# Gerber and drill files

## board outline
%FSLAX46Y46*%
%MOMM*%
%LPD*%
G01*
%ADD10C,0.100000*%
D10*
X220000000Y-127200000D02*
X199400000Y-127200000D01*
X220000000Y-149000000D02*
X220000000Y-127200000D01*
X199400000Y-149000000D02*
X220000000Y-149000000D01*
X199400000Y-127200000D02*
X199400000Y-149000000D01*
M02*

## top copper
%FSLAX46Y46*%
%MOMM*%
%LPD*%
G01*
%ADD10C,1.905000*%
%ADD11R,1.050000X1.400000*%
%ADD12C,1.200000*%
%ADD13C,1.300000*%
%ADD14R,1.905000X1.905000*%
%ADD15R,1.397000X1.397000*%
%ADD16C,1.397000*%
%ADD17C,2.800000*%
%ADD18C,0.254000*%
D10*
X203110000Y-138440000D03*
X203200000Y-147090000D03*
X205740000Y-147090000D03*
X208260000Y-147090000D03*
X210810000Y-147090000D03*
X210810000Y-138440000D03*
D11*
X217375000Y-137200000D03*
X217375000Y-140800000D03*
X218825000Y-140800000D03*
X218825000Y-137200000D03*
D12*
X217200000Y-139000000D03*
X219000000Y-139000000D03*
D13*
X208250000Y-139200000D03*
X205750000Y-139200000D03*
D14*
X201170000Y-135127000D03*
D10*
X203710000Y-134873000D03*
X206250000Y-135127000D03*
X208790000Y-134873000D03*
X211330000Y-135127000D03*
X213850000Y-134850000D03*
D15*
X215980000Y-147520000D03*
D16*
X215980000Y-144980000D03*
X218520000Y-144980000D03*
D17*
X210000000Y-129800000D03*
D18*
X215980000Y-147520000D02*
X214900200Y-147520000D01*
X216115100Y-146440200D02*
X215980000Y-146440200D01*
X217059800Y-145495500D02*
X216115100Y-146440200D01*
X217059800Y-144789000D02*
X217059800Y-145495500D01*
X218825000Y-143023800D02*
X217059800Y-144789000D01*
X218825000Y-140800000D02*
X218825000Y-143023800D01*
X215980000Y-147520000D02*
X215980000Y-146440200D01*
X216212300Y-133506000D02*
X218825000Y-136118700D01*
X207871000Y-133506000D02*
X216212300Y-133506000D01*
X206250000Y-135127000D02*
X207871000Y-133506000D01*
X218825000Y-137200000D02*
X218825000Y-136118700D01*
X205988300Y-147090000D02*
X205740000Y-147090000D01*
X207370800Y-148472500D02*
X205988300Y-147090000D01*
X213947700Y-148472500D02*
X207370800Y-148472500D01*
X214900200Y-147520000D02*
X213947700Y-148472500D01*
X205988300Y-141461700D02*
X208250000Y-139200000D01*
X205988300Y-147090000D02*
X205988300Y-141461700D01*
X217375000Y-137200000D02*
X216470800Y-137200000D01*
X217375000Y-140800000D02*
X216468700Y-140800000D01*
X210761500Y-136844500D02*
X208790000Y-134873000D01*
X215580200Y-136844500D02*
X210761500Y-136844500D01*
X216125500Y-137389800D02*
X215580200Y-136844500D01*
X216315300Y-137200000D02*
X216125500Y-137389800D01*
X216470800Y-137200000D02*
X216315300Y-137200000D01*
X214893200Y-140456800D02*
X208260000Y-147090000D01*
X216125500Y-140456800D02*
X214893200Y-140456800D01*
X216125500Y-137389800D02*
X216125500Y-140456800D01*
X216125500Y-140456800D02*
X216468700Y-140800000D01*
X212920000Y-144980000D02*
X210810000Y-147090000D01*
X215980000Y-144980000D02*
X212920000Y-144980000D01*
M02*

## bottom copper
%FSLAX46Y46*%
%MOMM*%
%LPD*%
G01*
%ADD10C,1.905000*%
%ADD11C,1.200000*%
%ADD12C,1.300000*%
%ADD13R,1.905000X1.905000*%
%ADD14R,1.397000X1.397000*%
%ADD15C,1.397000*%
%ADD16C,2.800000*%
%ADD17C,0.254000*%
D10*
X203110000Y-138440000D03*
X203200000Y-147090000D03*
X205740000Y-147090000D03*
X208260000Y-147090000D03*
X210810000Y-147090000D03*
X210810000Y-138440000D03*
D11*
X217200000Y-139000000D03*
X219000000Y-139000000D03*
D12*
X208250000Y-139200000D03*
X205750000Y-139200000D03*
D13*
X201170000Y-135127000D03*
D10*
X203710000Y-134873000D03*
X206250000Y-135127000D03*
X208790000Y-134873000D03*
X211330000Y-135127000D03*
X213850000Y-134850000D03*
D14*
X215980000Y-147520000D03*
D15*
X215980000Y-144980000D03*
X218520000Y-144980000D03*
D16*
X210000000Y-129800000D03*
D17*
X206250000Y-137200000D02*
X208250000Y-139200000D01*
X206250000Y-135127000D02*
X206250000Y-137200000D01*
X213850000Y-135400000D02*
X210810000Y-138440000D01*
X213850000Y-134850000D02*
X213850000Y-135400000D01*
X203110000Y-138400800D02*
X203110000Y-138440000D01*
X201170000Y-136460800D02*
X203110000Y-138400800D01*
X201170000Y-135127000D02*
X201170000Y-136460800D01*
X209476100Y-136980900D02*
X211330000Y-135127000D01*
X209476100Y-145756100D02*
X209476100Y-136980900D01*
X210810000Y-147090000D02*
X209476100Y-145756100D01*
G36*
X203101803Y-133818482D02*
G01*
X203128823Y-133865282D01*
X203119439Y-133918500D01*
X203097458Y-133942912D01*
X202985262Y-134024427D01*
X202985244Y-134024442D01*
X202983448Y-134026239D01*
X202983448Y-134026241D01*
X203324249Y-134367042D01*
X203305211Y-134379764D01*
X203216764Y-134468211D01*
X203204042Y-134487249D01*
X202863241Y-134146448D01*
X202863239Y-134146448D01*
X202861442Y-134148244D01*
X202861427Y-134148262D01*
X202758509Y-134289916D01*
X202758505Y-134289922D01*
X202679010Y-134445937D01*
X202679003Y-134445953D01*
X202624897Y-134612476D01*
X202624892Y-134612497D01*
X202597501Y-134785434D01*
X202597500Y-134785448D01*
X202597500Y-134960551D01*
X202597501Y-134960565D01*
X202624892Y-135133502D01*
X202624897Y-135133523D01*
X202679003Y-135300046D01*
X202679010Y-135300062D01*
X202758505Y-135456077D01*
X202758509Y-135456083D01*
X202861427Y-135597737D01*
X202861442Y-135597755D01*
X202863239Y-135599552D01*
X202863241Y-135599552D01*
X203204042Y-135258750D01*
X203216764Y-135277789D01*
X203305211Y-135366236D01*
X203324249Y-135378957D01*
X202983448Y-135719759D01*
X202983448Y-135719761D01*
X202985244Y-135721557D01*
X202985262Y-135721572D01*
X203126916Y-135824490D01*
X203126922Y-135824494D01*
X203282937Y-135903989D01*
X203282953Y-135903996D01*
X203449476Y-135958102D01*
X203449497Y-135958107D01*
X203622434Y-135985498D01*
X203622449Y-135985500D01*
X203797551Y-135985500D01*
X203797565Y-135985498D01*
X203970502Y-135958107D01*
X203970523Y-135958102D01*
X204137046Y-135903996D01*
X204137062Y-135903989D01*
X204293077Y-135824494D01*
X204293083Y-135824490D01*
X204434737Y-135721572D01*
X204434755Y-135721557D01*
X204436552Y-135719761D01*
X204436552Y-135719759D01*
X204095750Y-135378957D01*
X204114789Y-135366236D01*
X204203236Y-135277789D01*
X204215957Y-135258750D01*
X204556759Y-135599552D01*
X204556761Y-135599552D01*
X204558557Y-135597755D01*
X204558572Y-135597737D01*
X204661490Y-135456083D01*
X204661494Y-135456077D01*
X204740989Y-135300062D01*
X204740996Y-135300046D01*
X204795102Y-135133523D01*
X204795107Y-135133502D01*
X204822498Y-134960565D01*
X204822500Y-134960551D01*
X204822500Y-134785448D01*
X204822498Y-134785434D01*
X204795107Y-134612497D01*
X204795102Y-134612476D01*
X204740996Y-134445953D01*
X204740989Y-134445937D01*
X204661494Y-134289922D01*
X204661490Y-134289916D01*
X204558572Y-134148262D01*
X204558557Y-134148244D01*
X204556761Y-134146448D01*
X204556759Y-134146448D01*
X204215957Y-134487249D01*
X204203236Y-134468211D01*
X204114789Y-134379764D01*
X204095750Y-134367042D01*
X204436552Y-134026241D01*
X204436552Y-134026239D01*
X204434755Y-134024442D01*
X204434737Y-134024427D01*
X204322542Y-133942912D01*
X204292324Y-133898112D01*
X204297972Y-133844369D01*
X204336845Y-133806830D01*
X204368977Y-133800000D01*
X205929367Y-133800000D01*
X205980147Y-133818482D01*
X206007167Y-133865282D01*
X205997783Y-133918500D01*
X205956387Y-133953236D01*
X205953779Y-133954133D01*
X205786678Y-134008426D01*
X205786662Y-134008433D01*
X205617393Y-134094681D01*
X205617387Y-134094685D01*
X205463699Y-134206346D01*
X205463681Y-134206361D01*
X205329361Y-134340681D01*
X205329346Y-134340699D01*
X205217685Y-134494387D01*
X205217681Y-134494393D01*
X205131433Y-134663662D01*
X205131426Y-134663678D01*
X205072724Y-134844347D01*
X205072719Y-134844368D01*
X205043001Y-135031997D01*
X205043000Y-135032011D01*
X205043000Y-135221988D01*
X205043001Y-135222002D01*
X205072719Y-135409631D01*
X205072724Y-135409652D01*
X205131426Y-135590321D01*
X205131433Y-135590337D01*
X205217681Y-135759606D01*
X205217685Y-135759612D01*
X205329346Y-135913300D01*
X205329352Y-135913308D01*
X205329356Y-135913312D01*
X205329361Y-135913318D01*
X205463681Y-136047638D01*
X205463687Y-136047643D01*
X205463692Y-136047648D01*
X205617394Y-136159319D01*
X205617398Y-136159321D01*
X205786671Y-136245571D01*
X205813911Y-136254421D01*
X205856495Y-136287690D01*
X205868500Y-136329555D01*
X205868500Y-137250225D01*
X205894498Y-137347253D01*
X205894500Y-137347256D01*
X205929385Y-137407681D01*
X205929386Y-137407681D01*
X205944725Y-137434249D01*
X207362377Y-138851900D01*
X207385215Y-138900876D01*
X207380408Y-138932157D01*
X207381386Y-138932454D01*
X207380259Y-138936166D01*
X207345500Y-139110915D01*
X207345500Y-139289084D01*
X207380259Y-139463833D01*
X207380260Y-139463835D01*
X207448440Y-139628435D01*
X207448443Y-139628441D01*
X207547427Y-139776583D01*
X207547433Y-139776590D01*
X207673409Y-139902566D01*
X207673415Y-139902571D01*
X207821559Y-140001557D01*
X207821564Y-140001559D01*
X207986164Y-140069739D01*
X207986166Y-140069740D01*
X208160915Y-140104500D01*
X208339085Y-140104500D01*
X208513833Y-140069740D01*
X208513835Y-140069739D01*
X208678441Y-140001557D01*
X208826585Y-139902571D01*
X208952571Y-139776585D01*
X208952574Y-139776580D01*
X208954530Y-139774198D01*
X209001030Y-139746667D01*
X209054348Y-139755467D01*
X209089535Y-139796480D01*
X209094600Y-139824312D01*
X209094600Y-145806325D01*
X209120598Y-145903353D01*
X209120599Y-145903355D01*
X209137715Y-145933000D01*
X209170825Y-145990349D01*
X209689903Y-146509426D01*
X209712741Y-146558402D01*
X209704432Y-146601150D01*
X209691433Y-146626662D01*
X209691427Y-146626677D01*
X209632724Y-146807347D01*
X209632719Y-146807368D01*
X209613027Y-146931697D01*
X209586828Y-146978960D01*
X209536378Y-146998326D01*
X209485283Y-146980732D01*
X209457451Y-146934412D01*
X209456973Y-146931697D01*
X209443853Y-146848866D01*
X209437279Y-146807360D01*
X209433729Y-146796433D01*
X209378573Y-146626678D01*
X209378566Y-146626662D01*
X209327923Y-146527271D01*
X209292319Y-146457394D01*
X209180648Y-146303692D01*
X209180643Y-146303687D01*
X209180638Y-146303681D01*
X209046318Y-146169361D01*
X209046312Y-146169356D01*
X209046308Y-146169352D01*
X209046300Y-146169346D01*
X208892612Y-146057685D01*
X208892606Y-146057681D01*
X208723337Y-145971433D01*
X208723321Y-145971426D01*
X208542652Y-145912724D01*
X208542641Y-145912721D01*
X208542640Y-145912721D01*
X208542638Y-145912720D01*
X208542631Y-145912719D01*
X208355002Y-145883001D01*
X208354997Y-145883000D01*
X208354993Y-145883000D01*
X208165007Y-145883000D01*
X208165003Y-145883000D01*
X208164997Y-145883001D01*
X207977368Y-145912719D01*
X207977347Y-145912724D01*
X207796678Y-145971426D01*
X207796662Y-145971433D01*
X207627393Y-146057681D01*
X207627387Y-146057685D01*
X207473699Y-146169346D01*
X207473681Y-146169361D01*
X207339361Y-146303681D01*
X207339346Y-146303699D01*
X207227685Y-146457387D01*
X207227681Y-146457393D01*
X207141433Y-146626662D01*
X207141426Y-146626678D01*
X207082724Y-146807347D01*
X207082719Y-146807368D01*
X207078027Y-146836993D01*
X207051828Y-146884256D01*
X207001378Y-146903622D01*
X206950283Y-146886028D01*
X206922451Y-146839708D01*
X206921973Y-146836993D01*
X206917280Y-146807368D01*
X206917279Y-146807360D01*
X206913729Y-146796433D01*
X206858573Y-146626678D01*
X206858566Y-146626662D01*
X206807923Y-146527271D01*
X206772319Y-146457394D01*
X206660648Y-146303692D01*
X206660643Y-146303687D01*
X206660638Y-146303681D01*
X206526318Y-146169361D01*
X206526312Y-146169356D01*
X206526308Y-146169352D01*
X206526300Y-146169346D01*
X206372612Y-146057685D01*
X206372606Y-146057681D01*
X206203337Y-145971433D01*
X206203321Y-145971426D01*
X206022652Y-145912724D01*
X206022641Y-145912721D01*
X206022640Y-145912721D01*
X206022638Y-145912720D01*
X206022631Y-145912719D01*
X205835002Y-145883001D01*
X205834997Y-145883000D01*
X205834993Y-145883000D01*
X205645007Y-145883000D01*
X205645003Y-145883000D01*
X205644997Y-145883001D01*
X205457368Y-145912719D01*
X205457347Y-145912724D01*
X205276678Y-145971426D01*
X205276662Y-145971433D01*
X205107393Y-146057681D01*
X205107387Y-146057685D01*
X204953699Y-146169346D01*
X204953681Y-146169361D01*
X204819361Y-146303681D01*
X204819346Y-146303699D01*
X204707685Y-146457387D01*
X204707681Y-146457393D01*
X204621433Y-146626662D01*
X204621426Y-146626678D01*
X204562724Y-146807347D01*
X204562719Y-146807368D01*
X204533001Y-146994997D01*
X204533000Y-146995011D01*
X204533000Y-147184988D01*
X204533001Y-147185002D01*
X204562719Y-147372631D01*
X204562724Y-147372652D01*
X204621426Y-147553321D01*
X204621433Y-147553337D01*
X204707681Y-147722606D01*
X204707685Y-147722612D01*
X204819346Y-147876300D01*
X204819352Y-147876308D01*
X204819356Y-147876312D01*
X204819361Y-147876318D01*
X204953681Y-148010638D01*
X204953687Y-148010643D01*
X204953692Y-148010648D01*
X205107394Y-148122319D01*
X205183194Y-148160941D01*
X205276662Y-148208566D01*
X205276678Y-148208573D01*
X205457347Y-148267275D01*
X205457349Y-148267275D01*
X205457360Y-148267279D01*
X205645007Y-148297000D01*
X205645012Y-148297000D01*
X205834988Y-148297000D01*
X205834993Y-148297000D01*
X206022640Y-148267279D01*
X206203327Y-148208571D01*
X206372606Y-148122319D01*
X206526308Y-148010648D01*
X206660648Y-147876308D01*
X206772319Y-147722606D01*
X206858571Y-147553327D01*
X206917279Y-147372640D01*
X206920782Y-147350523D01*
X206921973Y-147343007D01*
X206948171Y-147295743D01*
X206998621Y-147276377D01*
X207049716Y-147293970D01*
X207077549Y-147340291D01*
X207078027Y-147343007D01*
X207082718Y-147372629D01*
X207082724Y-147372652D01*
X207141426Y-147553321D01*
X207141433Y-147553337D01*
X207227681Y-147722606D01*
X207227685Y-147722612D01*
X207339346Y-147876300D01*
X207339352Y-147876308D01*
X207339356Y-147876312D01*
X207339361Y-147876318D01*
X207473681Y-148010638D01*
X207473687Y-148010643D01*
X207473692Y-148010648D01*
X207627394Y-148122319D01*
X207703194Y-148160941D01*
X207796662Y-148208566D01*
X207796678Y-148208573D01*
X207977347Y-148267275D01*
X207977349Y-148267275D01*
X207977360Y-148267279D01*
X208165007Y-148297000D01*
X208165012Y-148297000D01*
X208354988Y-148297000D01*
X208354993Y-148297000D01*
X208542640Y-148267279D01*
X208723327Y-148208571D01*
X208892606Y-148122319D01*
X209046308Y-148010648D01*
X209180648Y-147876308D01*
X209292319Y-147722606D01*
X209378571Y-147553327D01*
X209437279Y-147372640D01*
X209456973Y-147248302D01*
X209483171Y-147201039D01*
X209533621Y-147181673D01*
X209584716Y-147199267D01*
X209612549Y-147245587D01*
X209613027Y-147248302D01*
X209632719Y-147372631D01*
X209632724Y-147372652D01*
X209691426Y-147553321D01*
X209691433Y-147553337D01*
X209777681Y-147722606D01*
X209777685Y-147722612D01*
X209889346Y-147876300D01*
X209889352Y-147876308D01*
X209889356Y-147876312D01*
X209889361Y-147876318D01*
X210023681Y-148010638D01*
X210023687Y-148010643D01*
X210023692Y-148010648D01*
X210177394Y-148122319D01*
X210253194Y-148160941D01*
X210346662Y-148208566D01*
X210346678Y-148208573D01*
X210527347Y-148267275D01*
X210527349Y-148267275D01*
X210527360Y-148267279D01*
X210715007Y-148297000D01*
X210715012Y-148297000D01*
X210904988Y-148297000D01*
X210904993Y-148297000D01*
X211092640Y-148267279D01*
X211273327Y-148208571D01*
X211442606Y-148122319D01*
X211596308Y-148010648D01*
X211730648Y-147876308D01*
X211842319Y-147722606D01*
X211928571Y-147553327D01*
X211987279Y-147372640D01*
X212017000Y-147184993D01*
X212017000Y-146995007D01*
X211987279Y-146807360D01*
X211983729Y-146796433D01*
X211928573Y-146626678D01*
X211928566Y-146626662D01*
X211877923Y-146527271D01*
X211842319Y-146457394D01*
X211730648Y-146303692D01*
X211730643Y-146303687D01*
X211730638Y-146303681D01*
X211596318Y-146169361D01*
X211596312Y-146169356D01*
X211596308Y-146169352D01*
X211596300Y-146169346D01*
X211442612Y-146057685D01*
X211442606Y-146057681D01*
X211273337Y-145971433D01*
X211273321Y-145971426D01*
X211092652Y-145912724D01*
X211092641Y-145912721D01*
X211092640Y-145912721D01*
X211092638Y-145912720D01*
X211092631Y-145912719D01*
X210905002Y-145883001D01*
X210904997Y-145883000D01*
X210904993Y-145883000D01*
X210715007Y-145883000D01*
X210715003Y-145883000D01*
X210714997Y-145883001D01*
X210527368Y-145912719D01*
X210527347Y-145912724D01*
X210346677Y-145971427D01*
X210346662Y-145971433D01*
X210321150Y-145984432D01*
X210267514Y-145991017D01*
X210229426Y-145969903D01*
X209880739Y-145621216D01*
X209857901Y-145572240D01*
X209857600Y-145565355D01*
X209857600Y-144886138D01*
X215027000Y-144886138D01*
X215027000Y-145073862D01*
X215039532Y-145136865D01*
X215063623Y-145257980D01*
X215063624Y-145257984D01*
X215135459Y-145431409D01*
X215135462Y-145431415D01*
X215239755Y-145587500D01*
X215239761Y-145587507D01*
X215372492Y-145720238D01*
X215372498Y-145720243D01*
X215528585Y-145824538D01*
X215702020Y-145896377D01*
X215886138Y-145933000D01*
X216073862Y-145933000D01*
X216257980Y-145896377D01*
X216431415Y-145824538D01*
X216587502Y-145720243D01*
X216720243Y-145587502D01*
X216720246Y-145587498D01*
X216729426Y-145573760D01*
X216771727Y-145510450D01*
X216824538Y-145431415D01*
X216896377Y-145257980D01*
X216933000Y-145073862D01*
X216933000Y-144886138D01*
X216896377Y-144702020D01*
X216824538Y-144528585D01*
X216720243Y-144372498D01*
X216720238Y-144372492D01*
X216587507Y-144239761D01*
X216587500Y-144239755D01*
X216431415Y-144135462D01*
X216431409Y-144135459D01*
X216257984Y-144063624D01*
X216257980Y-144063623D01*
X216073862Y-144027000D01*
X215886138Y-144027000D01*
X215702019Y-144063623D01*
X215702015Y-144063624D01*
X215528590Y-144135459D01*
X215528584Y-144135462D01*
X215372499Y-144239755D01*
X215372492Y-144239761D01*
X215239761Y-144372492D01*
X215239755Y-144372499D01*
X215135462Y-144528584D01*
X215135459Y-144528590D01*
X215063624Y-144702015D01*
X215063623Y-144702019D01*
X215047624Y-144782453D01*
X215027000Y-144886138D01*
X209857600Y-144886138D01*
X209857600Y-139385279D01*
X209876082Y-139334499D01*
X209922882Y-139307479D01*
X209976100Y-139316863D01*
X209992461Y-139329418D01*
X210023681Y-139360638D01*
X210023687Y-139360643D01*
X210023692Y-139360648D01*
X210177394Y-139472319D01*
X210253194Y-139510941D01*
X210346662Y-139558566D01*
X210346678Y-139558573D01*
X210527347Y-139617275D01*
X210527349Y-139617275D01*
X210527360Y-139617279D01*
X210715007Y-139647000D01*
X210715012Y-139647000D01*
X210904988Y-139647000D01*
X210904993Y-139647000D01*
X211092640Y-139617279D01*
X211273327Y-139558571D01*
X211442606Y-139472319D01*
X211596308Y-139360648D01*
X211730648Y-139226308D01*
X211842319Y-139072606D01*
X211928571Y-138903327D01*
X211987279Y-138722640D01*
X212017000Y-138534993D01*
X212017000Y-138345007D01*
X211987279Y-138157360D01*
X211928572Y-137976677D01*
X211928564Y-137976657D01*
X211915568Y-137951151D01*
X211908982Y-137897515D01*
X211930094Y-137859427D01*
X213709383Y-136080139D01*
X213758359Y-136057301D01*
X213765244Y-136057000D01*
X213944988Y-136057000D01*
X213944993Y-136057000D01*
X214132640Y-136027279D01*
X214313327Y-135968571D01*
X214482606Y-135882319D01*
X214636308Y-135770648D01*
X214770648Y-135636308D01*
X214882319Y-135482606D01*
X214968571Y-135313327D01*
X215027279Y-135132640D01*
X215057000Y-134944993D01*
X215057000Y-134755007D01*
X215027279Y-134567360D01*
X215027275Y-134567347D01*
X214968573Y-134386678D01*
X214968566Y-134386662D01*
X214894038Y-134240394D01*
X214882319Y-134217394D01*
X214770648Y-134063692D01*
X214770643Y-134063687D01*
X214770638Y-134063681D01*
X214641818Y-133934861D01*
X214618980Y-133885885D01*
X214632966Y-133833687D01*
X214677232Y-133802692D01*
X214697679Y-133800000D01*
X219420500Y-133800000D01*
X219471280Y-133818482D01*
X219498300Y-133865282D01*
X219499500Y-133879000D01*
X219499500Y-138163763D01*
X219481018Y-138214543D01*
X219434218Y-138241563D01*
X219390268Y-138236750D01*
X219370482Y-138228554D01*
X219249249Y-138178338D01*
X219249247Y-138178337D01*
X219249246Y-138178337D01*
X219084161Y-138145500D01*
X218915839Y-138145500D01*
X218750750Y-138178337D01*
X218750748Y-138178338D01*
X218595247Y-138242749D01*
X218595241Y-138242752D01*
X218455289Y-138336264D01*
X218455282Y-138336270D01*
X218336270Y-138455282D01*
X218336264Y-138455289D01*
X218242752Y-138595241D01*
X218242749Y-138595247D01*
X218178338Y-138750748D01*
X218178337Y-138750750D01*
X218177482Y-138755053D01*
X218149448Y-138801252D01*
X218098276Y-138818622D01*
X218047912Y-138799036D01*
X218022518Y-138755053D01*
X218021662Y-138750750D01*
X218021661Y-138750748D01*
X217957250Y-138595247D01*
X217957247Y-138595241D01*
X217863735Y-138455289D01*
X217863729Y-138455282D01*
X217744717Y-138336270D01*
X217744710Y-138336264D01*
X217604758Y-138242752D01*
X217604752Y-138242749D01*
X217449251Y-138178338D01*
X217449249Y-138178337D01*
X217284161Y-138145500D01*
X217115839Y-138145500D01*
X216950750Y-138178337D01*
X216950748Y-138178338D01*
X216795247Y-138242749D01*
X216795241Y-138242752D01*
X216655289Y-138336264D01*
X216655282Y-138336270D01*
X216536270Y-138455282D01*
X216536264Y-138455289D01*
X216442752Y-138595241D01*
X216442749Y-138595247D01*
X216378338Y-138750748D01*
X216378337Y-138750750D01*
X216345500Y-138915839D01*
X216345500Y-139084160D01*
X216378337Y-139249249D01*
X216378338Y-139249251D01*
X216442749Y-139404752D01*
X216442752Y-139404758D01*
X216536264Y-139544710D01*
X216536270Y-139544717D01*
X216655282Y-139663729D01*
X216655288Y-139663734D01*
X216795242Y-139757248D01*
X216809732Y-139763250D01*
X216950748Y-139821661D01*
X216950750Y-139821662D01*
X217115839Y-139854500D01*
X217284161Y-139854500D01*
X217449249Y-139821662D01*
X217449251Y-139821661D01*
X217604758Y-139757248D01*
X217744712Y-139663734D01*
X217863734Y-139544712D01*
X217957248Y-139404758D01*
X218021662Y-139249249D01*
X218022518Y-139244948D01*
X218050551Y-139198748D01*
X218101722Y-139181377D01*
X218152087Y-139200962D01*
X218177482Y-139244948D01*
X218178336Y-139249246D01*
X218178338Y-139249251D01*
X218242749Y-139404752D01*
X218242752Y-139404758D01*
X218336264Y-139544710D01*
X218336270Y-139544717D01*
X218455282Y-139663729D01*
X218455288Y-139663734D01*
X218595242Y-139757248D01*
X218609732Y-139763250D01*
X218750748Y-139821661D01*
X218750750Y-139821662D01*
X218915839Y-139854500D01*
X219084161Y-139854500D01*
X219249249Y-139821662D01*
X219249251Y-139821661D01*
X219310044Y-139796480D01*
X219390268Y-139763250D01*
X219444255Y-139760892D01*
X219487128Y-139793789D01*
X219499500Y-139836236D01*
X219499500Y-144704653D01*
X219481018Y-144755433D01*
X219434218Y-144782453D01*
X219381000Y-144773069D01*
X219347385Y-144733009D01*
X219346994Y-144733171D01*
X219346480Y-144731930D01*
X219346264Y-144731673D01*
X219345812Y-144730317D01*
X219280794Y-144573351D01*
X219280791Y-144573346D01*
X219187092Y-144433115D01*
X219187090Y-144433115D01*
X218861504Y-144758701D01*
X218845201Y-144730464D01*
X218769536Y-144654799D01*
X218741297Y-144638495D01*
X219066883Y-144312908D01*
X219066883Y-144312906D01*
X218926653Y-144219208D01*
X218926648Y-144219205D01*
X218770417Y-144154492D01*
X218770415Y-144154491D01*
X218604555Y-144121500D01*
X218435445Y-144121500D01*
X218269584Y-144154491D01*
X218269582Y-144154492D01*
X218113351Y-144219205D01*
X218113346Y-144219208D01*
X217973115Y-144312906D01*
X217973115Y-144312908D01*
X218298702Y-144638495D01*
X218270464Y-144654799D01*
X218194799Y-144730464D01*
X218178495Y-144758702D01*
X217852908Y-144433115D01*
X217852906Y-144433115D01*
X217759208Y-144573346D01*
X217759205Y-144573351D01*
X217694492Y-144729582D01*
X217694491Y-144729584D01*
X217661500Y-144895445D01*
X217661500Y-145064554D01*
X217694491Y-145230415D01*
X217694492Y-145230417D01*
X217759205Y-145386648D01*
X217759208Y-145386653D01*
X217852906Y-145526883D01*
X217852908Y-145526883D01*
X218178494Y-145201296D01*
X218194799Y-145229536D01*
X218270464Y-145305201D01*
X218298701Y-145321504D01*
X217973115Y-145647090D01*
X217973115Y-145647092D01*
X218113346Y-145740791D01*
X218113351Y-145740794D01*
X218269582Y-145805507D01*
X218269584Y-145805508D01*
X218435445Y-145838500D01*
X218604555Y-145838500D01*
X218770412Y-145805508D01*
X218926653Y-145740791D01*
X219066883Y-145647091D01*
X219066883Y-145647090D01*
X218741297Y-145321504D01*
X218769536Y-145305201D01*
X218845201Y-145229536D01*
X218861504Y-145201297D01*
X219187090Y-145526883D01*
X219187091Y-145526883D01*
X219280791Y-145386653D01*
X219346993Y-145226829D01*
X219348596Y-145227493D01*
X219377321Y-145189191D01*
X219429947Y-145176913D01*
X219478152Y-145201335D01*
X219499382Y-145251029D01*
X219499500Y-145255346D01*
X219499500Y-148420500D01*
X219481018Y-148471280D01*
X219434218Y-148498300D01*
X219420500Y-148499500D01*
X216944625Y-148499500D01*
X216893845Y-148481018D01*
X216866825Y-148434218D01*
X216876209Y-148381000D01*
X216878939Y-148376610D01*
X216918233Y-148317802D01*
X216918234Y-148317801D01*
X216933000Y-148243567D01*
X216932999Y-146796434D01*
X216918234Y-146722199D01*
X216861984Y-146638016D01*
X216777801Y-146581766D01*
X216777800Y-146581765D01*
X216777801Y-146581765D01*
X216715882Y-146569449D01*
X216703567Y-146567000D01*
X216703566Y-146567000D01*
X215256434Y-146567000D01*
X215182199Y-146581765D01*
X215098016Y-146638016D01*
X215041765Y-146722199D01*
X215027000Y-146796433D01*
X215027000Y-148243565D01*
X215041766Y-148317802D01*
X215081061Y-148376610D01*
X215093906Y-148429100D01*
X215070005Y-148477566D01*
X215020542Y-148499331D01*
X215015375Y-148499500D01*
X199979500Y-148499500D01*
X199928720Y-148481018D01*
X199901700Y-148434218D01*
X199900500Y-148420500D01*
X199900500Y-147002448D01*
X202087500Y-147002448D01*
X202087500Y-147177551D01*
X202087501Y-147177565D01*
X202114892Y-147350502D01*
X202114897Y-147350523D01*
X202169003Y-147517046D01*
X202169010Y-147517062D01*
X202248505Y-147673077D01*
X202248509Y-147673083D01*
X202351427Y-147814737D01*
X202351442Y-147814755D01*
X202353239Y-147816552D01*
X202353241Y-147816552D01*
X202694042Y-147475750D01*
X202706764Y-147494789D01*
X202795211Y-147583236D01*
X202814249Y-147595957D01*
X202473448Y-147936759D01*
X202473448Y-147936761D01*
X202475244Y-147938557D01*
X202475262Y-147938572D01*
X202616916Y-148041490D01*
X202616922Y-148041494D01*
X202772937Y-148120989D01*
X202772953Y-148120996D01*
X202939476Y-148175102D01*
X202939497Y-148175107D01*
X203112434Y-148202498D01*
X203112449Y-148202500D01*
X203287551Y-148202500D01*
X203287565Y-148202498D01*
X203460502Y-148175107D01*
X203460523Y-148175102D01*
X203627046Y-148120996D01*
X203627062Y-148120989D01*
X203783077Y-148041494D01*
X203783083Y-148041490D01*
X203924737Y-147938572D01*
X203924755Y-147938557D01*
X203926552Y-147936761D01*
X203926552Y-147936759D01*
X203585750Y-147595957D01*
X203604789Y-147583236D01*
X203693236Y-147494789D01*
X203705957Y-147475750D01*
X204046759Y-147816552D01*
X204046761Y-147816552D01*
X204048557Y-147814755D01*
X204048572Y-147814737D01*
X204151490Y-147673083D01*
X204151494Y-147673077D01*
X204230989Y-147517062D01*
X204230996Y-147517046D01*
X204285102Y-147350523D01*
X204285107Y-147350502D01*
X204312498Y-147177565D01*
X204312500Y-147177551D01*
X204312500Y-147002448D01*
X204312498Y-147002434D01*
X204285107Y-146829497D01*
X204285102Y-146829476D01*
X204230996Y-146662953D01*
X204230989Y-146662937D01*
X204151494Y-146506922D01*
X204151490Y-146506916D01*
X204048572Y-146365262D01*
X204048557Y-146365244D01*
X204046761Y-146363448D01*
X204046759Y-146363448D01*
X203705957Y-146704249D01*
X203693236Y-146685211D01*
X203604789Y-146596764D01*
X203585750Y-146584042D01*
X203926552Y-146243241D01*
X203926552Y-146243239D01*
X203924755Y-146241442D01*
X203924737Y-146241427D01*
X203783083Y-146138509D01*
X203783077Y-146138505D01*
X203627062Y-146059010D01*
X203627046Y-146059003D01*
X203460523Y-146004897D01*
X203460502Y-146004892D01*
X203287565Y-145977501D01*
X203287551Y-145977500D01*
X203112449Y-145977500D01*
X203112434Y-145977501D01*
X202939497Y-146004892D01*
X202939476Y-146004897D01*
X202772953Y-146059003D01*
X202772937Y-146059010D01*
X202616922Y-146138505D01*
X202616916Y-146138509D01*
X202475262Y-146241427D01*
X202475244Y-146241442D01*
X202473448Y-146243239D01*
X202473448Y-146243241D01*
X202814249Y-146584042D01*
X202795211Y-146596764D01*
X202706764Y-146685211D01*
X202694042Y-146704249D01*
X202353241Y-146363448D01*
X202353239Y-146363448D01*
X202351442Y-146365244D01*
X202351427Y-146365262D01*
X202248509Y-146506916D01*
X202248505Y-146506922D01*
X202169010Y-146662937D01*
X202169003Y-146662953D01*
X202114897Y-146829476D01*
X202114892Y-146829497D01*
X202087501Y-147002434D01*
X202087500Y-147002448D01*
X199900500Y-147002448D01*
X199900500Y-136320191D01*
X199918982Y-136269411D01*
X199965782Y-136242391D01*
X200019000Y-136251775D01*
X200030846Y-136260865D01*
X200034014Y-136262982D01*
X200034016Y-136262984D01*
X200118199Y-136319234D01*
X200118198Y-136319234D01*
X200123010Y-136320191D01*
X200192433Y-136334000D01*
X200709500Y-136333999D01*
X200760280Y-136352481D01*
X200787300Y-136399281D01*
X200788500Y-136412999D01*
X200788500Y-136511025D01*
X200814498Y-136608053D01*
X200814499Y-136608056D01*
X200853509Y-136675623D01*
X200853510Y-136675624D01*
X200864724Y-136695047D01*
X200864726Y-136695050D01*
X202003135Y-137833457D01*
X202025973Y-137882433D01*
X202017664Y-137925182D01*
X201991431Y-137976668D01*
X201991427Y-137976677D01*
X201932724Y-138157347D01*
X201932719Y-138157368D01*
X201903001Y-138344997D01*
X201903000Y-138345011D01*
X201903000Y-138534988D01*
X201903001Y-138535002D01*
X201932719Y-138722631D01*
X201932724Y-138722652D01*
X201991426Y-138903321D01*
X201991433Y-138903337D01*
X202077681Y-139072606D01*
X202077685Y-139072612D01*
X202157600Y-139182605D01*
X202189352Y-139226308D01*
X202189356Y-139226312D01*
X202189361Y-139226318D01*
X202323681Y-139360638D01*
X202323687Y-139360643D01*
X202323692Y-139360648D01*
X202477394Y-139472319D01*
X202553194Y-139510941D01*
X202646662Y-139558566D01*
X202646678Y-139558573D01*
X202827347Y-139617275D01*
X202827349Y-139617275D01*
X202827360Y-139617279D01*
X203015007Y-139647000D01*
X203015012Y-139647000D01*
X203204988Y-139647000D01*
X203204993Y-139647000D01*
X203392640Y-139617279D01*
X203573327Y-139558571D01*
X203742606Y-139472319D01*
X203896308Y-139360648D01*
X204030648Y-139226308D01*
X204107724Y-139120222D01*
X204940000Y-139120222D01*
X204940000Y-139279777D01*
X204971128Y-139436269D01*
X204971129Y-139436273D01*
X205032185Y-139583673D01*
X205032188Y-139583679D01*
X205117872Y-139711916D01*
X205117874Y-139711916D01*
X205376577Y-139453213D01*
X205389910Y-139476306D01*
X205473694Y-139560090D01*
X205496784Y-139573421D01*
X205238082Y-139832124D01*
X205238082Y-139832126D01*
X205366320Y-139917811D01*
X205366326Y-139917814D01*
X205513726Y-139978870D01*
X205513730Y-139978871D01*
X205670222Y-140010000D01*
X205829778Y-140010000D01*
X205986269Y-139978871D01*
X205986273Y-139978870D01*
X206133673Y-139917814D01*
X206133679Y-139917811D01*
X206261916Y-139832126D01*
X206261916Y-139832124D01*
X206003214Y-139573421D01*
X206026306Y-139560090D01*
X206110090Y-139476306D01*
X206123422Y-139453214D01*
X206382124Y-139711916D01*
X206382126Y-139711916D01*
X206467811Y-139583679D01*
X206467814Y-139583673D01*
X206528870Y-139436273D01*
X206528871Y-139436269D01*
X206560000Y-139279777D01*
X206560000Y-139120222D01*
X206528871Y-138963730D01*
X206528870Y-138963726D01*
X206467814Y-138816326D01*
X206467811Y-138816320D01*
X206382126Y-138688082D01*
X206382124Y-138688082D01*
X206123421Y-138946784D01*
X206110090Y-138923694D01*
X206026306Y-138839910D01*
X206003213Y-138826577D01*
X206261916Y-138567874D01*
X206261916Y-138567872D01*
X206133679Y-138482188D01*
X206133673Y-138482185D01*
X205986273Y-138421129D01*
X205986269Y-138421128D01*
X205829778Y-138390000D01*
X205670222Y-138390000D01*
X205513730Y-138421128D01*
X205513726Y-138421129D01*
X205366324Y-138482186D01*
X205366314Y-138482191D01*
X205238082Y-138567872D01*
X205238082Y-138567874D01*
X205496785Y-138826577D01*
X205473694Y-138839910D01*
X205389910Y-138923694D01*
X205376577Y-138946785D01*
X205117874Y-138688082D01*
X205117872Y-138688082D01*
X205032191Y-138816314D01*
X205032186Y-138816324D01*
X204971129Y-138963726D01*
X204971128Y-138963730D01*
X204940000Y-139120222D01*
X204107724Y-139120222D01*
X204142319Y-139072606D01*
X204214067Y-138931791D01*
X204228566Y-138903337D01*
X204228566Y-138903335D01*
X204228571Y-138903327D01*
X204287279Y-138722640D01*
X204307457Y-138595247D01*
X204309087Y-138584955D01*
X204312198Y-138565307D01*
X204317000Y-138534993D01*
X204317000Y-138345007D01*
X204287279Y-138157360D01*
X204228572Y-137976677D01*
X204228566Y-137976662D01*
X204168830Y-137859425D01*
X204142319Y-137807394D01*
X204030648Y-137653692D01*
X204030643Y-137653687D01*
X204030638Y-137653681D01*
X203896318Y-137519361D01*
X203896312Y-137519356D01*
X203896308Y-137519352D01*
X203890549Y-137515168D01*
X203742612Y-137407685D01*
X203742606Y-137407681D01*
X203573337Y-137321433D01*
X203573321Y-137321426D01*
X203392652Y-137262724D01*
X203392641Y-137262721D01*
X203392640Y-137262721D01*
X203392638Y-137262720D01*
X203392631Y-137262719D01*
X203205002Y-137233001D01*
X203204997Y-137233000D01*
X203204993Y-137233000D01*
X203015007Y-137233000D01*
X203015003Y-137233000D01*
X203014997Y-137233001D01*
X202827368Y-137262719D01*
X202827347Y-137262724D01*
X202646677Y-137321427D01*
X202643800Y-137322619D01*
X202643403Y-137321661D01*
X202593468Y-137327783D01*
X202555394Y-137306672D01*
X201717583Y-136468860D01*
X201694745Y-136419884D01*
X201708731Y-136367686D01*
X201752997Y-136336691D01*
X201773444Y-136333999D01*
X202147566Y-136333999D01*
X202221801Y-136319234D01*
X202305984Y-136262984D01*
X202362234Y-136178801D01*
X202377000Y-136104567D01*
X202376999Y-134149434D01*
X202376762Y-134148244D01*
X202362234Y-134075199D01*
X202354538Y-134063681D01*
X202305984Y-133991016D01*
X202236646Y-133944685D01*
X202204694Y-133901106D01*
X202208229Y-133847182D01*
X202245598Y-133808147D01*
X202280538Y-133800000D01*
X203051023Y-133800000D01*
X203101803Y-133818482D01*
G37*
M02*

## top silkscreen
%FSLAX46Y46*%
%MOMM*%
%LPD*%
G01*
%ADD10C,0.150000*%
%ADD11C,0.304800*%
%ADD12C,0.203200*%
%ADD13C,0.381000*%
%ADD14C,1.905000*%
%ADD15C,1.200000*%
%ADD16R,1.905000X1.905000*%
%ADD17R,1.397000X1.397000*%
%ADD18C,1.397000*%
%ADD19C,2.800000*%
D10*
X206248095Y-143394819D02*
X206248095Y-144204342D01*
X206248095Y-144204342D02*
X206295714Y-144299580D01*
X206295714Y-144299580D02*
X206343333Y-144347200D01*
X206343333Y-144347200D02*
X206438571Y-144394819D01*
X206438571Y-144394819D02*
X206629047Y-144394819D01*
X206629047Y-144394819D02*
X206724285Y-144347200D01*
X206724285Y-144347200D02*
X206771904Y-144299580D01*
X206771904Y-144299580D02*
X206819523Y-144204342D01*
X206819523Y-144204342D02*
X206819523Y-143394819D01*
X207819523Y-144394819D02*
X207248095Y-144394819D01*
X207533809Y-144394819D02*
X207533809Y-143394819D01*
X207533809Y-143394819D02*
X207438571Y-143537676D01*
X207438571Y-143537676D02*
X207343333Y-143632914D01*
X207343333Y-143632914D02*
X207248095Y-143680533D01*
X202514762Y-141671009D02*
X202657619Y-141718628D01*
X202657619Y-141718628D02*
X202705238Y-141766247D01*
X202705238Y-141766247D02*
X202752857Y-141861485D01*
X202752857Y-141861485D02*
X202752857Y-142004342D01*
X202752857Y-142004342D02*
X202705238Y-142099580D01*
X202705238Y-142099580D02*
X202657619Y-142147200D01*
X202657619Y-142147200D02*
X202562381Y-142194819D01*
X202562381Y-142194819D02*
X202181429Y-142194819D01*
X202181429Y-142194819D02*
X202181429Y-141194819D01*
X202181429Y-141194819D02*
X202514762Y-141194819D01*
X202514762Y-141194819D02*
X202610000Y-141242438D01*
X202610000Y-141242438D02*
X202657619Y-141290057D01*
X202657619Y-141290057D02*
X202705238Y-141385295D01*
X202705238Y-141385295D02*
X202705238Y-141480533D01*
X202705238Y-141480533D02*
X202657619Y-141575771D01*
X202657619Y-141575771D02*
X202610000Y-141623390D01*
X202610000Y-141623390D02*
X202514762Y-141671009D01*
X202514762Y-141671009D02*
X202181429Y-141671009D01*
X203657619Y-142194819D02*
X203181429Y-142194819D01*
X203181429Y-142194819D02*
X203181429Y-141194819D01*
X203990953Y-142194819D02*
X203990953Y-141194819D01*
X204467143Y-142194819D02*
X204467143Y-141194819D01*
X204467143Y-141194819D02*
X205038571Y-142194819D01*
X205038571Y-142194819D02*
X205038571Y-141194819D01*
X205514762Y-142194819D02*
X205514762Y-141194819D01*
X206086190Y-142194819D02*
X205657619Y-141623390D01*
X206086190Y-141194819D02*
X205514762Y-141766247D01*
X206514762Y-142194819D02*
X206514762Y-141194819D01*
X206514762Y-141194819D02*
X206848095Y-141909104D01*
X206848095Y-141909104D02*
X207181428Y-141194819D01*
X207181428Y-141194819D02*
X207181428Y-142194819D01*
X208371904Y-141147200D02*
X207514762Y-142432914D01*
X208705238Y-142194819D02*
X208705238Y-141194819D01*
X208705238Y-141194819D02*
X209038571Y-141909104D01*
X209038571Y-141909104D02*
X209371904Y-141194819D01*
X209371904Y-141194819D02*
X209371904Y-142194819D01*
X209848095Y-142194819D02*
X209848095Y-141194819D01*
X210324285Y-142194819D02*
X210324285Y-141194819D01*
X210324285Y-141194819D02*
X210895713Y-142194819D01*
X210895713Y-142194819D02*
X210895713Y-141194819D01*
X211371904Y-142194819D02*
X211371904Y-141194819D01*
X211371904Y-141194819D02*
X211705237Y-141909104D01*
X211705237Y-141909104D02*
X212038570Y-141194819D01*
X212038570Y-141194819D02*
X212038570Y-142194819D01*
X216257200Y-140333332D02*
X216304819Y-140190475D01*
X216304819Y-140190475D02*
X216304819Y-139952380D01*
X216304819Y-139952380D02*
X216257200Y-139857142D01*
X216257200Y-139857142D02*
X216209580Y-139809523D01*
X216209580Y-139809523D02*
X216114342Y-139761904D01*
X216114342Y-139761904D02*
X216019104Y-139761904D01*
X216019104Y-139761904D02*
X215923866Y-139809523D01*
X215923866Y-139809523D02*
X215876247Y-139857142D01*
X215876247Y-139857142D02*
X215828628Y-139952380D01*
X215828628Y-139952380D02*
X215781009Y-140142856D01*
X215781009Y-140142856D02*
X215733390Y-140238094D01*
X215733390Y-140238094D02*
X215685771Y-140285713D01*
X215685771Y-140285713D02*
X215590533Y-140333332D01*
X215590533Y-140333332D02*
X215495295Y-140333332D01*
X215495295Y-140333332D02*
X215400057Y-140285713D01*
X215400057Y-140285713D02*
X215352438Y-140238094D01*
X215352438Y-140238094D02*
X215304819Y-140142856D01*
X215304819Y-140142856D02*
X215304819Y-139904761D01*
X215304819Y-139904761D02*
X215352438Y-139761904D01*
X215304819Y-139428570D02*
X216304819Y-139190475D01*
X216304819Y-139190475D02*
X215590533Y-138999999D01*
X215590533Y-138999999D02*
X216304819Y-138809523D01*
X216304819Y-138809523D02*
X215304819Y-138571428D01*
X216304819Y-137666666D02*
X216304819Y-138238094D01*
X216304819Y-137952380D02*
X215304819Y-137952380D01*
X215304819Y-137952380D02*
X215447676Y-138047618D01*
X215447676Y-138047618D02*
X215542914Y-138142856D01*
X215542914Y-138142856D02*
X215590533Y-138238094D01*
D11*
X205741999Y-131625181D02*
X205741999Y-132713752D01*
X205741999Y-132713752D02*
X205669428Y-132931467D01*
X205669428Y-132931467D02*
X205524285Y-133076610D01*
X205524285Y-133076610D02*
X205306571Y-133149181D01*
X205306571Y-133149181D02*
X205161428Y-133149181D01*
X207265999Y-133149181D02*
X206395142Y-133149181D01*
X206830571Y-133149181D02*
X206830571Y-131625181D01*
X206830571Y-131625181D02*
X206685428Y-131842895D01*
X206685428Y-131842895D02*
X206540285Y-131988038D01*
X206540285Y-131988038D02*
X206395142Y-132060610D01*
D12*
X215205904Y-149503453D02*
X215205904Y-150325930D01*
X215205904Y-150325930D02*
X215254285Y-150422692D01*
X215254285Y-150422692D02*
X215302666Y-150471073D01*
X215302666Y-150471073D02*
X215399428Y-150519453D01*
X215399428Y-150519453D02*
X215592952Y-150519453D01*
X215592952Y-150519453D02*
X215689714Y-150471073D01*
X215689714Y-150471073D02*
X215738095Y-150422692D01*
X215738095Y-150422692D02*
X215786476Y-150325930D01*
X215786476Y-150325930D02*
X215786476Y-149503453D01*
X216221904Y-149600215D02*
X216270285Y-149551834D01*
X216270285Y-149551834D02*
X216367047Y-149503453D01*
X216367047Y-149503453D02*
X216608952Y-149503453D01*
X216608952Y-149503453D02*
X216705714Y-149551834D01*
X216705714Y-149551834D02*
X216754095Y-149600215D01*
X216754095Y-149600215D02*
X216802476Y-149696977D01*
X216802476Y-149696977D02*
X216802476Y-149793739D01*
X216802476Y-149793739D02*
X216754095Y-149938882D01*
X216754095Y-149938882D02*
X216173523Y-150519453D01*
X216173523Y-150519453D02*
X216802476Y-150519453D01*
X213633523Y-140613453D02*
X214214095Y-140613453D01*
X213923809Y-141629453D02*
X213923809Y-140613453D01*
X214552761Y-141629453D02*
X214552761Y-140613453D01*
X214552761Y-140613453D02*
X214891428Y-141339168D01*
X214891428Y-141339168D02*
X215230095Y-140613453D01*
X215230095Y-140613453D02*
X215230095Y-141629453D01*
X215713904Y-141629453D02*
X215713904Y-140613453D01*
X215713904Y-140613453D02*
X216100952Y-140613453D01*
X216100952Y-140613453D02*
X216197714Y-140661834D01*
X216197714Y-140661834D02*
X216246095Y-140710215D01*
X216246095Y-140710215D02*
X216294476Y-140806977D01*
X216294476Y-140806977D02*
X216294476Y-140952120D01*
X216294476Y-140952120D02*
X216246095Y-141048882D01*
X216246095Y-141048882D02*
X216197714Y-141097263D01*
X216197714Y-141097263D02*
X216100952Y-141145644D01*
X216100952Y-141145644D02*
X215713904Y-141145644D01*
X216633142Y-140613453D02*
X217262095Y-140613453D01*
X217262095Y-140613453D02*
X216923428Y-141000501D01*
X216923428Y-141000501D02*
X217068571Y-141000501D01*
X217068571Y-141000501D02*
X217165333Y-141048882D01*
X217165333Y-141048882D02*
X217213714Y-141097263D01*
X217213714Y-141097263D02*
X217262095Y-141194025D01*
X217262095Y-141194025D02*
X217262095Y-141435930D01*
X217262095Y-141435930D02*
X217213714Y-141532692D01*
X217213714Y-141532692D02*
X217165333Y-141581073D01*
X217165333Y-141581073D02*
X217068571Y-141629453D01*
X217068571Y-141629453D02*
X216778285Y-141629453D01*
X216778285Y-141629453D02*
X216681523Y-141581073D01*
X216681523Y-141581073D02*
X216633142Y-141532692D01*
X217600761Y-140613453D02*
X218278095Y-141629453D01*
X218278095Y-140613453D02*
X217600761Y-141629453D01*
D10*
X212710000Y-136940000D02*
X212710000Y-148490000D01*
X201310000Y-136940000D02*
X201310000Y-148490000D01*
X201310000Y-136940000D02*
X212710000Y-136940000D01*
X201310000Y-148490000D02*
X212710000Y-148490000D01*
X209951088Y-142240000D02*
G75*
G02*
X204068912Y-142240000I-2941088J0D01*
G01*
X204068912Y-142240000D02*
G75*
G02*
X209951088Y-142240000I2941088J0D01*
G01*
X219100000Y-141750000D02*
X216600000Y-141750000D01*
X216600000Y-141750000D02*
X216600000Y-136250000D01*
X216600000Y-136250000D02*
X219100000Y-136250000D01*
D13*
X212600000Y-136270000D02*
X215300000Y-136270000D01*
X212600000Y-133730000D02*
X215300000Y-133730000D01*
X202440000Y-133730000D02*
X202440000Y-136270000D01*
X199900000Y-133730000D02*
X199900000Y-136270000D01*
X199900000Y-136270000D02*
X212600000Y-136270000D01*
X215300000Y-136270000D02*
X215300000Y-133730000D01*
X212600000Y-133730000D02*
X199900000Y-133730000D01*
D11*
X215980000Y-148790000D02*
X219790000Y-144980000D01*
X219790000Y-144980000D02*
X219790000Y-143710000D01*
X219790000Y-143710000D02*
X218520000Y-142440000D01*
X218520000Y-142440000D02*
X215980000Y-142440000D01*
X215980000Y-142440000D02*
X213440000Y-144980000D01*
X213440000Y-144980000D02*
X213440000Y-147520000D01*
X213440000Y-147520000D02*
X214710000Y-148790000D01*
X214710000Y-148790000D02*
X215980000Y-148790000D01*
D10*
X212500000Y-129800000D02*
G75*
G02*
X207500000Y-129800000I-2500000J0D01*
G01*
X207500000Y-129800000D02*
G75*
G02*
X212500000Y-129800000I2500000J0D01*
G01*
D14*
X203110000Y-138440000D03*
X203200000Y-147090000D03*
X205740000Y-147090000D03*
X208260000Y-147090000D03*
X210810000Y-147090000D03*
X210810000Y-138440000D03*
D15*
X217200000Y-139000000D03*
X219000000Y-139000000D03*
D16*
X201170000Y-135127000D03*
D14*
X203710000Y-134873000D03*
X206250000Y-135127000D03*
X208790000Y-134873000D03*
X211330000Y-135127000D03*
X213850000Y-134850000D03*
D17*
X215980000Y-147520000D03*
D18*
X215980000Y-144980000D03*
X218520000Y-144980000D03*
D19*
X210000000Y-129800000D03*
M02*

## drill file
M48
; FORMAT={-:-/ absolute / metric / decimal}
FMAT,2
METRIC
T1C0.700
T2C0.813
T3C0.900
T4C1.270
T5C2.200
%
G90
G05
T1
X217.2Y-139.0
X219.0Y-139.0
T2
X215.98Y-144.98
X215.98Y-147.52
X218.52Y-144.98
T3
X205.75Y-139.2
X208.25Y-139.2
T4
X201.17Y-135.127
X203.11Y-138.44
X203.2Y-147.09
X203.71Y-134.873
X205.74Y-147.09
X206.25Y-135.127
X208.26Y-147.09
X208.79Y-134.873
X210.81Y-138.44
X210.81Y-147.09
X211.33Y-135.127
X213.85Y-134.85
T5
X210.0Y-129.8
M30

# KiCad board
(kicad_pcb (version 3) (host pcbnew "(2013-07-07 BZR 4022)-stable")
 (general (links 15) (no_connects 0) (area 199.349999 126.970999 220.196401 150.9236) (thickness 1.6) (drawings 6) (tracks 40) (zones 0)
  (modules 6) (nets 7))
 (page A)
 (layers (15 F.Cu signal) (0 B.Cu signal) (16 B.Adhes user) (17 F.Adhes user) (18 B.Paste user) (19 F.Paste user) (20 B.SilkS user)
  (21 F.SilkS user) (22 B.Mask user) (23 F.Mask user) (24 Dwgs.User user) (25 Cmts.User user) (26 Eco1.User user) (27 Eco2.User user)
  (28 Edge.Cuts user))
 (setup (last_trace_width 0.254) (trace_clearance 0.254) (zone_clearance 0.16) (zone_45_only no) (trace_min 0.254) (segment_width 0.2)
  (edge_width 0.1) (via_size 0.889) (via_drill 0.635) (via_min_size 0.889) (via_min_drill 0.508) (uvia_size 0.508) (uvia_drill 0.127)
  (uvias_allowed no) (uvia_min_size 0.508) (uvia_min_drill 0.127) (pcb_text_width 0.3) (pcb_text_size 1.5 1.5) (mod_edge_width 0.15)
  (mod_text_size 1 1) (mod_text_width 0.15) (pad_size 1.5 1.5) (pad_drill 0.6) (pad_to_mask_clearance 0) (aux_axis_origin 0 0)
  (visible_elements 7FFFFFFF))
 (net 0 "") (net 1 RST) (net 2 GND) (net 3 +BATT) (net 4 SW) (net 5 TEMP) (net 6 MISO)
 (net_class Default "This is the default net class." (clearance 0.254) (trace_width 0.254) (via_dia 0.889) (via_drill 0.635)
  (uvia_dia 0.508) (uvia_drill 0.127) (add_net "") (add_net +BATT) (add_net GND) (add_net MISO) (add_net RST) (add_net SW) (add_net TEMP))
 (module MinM (layer F.Cu) (at 207.01 142.24)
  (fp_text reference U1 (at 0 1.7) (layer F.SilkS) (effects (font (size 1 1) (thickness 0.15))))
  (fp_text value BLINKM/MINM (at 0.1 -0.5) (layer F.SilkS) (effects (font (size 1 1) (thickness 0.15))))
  (fp_line (start 5.7 -5.3) (end 5.7 6.25) (layer F.SilkS) (width 0.15))
  (fp_line (start -5.7 -5.3) (end -5.7 6.25) (layer F.SilkS) (width 0.15))
  (fp_line (start -5.7 -5.3) (end 5.7 -5.3) (layer F.SilkS) (width 0.15))
  (fp_line (start -5.7 6.25) (end 5.7 6.25) (layer F.SilkS) (width 0.15))
  (fp_circle (center 0 0) (end -2.4 -1.7) (layer F.SilkS) (width 0.15))
  (pad 1 thru_hole circle (at -3.9 -3.8) (size 1.905 1.905) (drill 1.27) (layers *.Cu *.Mask F.SilkS) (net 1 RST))
  (pad 2 thru_hole circle (at -3.81 4.85) (size 1.905 1.905) (drill 1.27) (layers *.Cu *.Mask F.SilkS) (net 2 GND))
  (pad 3 thru_hole circle (at -1.27 4.85) (size 1.905 1.905) (drill 1.27) (layers *.Cu *.Mask F.SilkS) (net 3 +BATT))
  (pad 4 thru_hole circle (at 1.25 4.85) (size 1.905 1.905) (drill 1.27) (layers *.Cu *.Mask F.SilkS) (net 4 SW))
  (pad 5 thru_hole circle (at 3.8 4.85) (size 1.905 1.905) (drill 1.27) (layers *.Cu *.Mask F.SilkS) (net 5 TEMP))
  (pad 6 thru_hole circle (at 3.8 -3.8) (size 1.905 1.905) (drill 1.27) (layers *.Cu *.Mask F.SilkS) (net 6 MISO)))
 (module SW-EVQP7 (layer F.Cu) (at 218.1 139 90)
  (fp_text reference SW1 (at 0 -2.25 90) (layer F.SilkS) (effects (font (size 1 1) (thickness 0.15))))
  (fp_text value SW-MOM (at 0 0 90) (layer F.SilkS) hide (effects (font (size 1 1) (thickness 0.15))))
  (fp_line (start -2.75 1) (end -2.75 -1.5) (layer F.SilkS) (width 0.15))
  (fp_line (start -2.75 -1.5) (end 2.75 -1.5) (layer F.SilkS) (width 0.15))
  (fp_line (start 2.75 -1.5) (end 2.75 1) (layer F.SilkS) (width 0.15))
  (pad 1 smd rect (at 1.8 -0.725 90) (size 1.4 1.05) (layers F.Cu F.Paste F.Mask) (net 4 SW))
  (pad 1 smd rect (at -1.8 -0.725 90) (size 1.4 1.05) (layers F.Cu F.Paste F.Mask) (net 4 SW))
  (pad 2 smd rect (at -1.8 0.725 90) (size 1.4 1.05) (layers F.Cu F.Paste F.Mask) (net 3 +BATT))
  (pad 2 smd rect (at 1.8 0.725 90) (size 1.4 1.05) (layers F.Cu F.Paste F.Mask) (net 3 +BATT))
  (pad "" thru_hole circle (at 0 -0.9 90) (size 1.2 1.2) (drill 0.7) (layers *.Cu *.Mask F.SilkS))
  (pad "" thru_hole circle (at 0 0.9 90) (size 1.2 1.2) (drill 0.7) (layers *.Cu *.Mask F.SilkS)))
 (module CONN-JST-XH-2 (layer B.Cu) (at 207 130 180)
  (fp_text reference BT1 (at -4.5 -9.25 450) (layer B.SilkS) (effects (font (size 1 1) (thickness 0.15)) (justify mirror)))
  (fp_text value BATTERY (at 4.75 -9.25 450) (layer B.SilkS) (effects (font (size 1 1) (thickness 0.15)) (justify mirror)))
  (pad 1 thru_hole circle (at -1.25 -9.2 180) (size 1.3 1.3) (drill 0.9) (layers *.Cu *.Mask B.SilkS) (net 3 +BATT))
  (pad 2 thru_hole circle (at 1.25 -9.2 180) (size 1.3 1.3) (drill 0.9) (layers *.Cu *.Mask B.SilkS) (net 2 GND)))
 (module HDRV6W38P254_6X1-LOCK (layer F.Cu) (at 206.25 135)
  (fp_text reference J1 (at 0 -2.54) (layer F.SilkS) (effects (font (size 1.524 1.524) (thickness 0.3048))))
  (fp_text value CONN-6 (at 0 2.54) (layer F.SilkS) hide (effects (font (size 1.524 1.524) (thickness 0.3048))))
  (fp_line (start 6.35 1.27) (end 9.05 1.27) (layer F.SilkS) (width 0.381))
  (fp_line (start 6.35 -1.27) (end 9.05 -1.27) (layer F.SilkS) (width 0.381))
  (fp_line (start -3.81 -1.27) (end -3.81 1.27) (layer F.SilkS) (width 0.381))
  (fp_line (start -6.35 -1.27) (end -6.35 1.27) (layer F.SilkS) (width 0.381))
  (fp_line (start -6.35 1.27) (end 6.35 1.27) (layer F.SilkS) (width 0.381))
  (fp_line (start 9.05 1.27) (end 9.05 -1.27) (layer F.SilkS) (width 0.381))
  (fp_line (start 6.35 -1.27) (end -6.35 -1.27) (layer F.SilkS) (width 0.381))
  (pad 1 thru_hole rect (at -5.08 0.127) (size 1.905 1.905) (drill 1.27) (layers *.Cu *.Mask F.SilkS) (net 1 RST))
  (pad 2 thru_hole circle (at -2.54 -0.127) (size 1.905 1.905) (drill 1.27) (layers *.Cu *.Mask F.SilkS) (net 2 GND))
  (pad 3 thru_hole circle (at 0 0.127) (size 1.905 1.905) (drill 1.27) (layers *.Cu *.Mask F.SilkS) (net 3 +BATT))
  (pad 4 thru_hole circle (at 2.54 -0.127) (size 1.905 1.905) (drill 1.27) (layers *.Cu *.Mask F.SilkS) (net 4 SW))
  (pad 5 thru_hole circle (at 5.08 0.127) (size 1.905 1.905) (drill 1.27) (layers *.Cu *.Mask F.SilkS) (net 5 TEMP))
  (pad 6 thru_hole circle (at 7.6 -0.15) (size 1.905 1.905) (drill 1.27) (layers *.Cu *.Mask F.SilkS) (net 6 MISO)))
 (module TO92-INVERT (layer F.Cu) (at 217.25 146.25)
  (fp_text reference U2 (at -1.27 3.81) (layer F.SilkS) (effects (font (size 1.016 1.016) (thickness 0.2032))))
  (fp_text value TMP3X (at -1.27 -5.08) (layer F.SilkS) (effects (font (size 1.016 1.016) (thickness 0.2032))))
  (fp_line (start -1.27 2.54) (end 2.54 -1.27) (layer F.SilkS) (width 0.3048))
  (fp_line (start 2.54 -1.27) (end 2.54 -2.54) (layer F.SilkS) (width 0.3048))
  (fp_line (start 2.54 -2.54) (end 1.27 -3.81) (layer F.SilkS) (width 0.3048))
  (fp_line (start 1.27 -3.81) (end -1.27 -3.81) (layer F.SilkS) (width 0.3048))
  (fp_line (start -1.27 -3.81) (end -3.81 -1.27) (layer F.SilkS) (width 0.3048))
  (fp_line (start -3.81 -1.27) (end -3.81 1.27) (layer F.SilkS) (width 0.3048))
  (fp_line (start -3.81 1.27) (end -2.54 2.54) (layer F.SilkS) (width 0.3048))
  (fp_line (start -2.54 2.54) (end -1.27 2.54) (layer F.SilkS) (width 0.3048))
  (pad 1 thru_hole rect (at -1.27 1.27) (size 1.397 1.397) (drill 0.8128) (layers *.Cu *.Mask F.SilkS) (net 3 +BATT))
  (pad 2 thru_hole circle (at -1.27 -1.27) (size 1.397 1.397) (drill 0.8128) (layers *.Cu *.Mask F.SilkS) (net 5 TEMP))
  (pad 3 thru_hole circle (at 1.27 -1.27) (size 1.397 1.397) (drill 0.8128) (layers *.Cu *.Mask F.SilkS) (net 2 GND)))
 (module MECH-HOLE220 (layer F.Cu) (at 210 129.8)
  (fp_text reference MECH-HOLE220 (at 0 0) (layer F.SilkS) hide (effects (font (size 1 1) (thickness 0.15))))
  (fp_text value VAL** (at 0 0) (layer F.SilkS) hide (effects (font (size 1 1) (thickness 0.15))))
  (fp_circle (center 0 0) (end 2.5 0) (layer F.SilkS) (width 0.15))
  (pad "" thru_hole circle (at 0 0) (size 2.8 2.8) (drill 2.2) (layers *.Cu *.Mask F.SilkS)))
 (gr_line (start 220 127.2) (end 199.4 127.2) (angle 90) (layer Edge.Cuts) (width 0.1))
 (gr_line (start 220 149) (end 220 127.2) (angle 90) (layer Edge.Cuts) (width 0.1))
 (gr_line (start 199.4 149) (end 220 149) (angle 90) (layer Edge.Cuts) (width 0.1))
 (gr_line (start 199.4 127.2) (end 199.4 149) (angle 90) (layer Edge.Cuts) (width 0.1))
 (segment (start 215.98 147.52) (end 214.9002 147.52) (width 0.254) (layer F.Cu) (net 3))
 (segment (start 206.25 137.2) (end 208.25 139.2) (width 0.254) (layer B.Cu) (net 3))
 (segment (start 206.25 135.127) (end 206.25 137.2) (width 0.254) (layer B.Cu) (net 3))
 (segment (start 216.1151 146.4402) (end 215.98 146.4402) (width 0.254) (layer F.Cu) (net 3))
 (segment (start 217.0598 145.4955) (end 216.1151 146.4402) (width 0.254) (layer F.Cu) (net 3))
 (segment (start 217.0598 144.789) (end 217.0598 145.4955) (width 0.254) (layer F.Cu) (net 3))
 (segment (start 218.825 143.0238) (end 217.0598 144.789) (width 0.254) (layer F.Cu) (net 3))
 (segment (start 218.825 140.8) (end 218.825 143.0238) (width 0.254) (layer F.Cu) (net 3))
 (segment (start 215.98 147.52) (end 215.98 146.4402) (width 0.254) (layer F.Cu) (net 3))
 (segment (start 216.2123 133.506) (end 218.825 136.1187) (width 0.254) (layer F.Cu) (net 3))
 (segment (start 207.871 133.506) (end 216.2123 133.506) (width 0.254) (layer F.Cu) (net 3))
 (segment (start 206.25 135.127) (end 207.871 133.506) (width 0.254) (layer F.Cu) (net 3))
 (segment (start 218.825 137.2) (end 218.825 136.1187) (width 0.254) (layer F.Cu) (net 3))
 (segment (start 205.9883 147.09) (end 205.74 147.09) (width 0.254) (layer F.Cu) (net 3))
 (segment (start 207.3708 148.4725) (end 205.9883 147.09) (width 0.254) (layer F.Cu) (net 3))
 (segment (start 213.9477 148.4725) (end 207.3708 148.4725) (width 0.254) (layer F.Cu) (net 3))
 (segment (start 214.9002 147.52) (end 213.9477 148.4725) (width 0.254) (layer F.Cu) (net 3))
 (segment (start 205.9883 141.4617) (end 208.25 139.2) (width 0.254) (layer F.Cu) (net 3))
 (segment (start 205.9883 147.09) (end 205.9883 141.4617) (width 0.254) (layer F.Cu) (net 3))
 (segment (start 213.85 135.4) (end 210.81 138.44) (width 0.254) (layer B.Cu) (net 6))
 (segment (start 213.85 134.85) (end 213.85 135.4) (width 0.254) (layer B.Cu) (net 6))
 (segment (start 203.11 138.4008) (end 203.11 138.44) (width 0.254) (layer B.Cu) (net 1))
 (segment (start 201.17 136.4608) (end 203.11 138.4008) (width 0.254) (layer B.Cu) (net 1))
 (segment (start 201.17 135.127) (end 201.17 136.4608) (width 0.254) (layer B.Cu) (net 1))
 (segment (start 217.375 137.2) (end 216.4708 137.2) (width 0.254) (layer F.Cu) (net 4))
 (segment (start 217.375 140.8) (end 216.4687 140.8) (width 0.254) (layer F.Cu) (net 4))
 (segment (start 210.7615 136.8445) (end 208.79 134.873) (width 0.254) (layer F.Cu) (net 4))
 (segment (start 215.5802 136.8445) (end 210.7615 136.8445) (width 0.254) (layer F.Cu) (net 4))
 (segment (start 216.1255 137.3898) (end 215.5802 136.8445) (width 0.254) (layer F.Cu) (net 4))
 (segment (start 216.3153 137.2) (end 216.1255 137.3898) (width 0.254) (layer F.Cu) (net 4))
 (segment (start 216.4708 137.2) (end 216.3153 137.2) (width 0.254) (layer F.Cu) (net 4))
 (segment (start 214.8932 140.4568) (end 208.26 147.09) (width 0.254) (layer F.Cu) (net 4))
 (segment (start 216.1255 140.4568) (end 214.8932 140.4568) (width 0.254) (layer F.Cu) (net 4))
 (segment (start 216.1255 137.3898) (end 216.1255 140.4568) (width 0.254) (layer F.Cu) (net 4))
 (segment (start 216.1255 140.4568) (end 216.4687 140.8) (width 0.254) (layer F.Cu) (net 4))
 (segment (start 212.92 144.98) (end 210.81 147.09) (width 0.254) (layer F.Cu) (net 5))
 (segment (start 215.98 144.98) (end 212.92 144.98) (width 0.254) (layer F.Cu) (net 5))
 (segment (start 209.4761 136.9809) (end 211.33 135.127) (width 0.254) (layer B.Cu) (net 5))
 (segment (start 209.4761 145.7561) (end 209.4761 136.9809) (width 0.254) (layer B.Cu) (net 5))
 (segment (start 210.81 147.09) (end 209.4761 145.7561) (width 0.254) (layer B.Cu) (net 5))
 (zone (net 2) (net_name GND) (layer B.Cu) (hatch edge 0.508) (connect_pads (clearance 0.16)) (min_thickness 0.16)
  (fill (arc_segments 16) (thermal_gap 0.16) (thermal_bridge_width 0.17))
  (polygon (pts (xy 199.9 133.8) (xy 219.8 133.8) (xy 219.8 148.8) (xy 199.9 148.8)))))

